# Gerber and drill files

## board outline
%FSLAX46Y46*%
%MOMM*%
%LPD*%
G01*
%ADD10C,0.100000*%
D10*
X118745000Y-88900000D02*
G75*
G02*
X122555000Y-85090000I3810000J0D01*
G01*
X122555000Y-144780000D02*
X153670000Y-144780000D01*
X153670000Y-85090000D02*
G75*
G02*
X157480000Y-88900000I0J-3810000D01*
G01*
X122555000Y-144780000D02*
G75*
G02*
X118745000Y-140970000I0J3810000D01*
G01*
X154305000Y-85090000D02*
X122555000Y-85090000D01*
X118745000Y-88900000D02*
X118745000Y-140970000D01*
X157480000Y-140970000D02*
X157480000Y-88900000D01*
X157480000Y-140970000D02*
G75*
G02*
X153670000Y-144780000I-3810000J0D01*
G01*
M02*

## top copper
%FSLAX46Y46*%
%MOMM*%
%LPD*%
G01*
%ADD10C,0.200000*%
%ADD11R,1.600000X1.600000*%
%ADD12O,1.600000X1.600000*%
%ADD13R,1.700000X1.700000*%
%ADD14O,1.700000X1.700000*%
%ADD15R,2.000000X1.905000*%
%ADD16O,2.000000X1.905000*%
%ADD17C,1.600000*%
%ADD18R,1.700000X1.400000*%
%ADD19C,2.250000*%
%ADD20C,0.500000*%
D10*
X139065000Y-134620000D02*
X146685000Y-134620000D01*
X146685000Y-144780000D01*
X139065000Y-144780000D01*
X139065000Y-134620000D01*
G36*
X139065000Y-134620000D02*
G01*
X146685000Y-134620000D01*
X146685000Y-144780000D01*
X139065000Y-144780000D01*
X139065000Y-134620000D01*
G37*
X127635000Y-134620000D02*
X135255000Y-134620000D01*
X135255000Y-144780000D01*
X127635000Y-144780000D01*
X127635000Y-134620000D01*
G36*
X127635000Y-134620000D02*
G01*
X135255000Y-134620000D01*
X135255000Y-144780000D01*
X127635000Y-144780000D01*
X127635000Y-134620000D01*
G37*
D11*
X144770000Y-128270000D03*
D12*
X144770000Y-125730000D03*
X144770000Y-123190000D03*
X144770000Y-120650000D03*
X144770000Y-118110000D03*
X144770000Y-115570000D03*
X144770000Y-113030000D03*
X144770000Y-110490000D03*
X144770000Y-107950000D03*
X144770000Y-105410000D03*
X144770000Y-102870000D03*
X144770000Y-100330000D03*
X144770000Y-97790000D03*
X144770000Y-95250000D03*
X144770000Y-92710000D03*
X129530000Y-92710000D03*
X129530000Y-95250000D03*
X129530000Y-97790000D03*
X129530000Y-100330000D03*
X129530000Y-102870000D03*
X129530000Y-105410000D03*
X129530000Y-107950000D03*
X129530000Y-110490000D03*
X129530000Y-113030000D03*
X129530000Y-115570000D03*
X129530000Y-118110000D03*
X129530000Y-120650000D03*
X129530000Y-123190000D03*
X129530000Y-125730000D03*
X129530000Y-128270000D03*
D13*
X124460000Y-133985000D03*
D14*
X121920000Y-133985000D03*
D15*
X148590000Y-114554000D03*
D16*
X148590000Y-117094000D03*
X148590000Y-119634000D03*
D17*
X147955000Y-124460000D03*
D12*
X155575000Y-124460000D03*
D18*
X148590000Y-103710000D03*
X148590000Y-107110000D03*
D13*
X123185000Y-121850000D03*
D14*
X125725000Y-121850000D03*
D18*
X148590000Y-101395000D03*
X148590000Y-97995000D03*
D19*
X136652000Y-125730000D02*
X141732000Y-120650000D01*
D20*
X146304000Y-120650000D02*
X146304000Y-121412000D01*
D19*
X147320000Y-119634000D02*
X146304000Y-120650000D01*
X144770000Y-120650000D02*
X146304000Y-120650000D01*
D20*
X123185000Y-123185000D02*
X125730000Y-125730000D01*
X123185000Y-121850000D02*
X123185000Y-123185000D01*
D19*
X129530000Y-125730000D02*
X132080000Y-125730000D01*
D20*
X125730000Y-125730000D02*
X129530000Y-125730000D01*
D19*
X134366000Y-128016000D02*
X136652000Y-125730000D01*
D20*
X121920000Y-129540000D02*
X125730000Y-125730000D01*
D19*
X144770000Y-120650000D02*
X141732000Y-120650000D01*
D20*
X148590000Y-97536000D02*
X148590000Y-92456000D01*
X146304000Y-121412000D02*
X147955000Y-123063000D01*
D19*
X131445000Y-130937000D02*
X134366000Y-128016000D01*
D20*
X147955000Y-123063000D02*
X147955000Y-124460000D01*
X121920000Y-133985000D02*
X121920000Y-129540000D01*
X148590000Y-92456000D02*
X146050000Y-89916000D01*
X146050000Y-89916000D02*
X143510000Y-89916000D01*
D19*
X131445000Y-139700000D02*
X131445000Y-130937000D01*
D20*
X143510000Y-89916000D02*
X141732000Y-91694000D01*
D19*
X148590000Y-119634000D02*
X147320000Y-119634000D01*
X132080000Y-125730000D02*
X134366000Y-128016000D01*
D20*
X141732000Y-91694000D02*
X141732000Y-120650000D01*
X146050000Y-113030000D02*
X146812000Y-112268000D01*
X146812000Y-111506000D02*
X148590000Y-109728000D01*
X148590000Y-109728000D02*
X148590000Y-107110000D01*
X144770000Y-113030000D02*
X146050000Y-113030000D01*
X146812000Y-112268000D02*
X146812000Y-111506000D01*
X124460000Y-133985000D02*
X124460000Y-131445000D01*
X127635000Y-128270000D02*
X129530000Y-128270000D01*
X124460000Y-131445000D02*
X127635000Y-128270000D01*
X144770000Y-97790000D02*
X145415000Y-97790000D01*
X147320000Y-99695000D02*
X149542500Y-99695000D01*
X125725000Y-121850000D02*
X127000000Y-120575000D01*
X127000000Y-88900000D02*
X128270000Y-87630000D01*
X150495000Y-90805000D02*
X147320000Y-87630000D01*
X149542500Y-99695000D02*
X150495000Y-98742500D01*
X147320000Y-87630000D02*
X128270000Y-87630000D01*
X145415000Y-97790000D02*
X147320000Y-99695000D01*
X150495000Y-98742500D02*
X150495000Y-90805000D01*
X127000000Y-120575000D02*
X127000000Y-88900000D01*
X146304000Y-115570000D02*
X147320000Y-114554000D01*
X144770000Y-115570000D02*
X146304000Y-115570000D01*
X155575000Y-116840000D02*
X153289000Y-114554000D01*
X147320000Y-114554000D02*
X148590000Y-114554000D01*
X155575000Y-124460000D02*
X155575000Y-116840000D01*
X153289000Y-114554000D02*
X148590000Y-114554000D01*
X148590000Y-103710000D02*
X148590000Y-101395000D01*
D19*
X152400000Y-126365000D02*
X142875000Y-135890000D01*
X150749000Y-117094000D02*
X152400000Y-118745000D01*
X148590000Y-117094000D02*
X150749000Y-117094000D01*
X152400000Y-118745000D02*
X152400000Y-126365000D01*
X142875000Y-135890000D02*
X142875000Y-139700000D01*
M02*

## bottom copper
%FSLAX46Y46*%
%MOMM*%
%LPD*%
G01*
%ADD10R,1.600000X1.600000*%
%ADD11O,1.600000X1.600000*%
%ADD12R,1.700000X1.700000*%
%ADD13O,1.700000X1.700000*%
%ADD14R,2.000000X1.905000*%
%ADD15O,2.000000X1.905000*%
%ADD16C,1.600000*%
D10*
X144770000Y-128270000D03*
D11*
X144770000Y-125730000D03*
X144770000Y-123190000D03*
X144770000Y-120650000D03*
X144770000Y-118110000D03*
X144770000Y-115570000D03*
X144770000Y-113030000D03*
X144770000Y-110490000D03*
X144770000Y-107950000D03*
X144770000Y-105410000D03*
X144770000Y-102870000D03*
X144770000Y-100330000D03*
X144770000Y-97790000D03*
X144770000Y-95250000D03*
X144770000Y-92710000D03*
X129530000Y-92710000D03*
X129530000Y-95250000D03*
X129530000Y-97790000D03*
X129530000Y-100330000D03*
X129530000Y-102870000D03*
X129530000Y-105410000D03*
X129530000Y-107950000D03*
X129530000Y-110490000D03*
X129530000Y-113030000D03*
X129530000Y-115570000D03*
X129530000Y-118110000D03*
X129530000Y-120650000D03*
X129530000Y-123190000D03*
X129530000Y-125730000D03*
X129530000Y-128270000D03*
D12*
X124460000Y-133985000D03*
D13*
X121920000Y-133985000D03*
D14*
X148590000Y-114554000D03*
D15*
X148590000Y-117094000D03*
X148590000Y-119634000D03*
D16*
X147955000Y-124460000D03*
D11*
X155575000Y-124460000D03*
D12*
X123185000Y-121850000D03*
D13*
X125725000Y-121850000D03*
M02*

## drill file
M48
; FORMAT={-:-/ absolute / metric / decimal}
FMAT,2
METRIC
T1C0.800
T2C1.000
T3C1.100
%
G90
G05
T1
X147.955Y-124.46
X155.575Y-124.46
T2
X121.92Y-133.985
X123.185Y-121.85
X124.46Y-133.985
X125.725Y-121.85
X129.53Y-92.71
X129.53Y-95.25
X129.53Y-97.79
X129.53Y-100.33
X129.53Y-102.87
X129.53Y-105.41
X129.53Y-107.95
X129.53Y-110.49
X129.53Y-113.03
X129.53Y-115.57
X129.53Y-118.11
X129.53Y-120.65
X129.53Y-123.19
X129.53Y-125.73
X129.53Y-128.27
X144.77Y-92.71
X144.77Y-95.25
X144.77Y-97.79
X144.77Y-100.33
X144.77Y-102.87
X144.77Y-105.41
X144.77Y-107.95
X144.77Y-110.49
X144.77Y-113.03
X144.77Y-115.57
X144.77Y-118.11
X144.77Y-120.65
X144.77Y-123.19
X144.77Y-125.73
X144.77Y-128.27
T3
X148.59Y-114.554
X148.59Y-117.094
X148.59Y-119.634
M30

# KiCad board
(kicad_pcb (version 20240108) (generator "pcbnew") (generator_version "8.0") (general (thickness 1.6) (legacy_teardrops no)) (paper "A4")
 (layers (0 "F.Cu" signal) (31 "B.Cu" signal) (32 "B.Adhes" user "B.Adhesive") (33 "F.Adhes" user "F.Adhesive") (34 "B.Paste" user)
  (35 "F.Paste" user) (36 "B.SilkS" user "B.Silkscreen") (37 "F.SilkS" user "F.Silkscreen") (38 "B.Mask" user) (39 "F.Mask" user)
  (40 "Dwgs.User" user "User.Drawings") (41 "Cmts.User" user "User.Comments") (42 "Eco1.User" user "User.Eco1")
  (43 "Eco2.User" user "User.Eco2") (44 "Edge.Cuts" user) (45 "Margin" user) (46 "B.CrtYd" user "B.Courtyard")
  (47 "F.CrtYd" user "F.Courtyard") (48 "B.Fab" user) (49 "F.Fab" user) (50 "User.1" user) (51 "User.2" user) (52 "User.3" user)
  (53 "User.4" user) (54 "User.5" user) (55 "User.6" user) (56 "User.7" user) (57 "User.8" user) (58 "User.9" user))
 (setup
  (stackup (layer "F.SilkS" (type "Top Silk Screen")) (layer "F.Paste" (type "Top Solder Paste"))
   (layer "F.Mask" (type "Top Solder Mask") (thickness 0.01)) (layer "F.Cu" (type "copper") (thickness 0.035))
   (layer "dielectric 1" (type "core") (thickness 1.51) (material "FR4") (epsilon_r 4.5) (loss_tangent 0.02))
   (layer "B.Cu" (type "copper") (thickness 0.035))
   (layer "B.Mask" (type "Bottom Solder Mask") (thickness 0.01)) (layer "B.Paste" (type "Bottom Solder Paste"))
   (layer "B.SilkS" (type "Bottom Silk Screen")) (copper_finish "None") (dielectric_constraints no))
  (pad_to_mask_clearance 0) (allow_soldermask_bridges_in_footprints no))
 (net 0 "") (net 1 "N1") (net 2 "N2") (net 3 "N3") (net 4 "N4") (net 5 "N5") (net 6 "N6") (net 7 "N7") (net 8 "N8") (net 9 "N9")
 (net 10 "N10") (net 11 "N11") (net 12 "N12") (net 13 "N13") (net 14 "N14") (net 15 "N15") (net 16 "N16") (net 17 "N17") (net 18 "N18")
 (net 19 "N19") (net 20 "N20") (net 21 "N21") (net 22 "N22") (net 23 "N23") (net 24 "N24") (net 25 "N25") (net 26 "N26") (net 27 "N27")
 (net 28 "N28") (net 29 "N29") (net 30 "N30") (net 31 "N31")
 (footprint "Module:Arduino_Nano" (layer "F.Cu") (at 144.77 128.27 180)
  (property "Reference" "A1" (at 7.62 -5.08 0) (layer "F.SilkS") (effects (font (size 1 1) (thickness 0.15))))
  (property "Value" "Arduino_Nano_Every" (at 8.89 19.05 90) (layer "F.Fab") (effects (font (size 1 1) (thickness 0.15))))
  (pad "1" thru_hole rect (at 0 0 180) (size 1.6 1.6) (drill 1) (layers "*.Cu" "*.Mask") (remove_unused_layers no) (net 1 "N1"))
  (pad "2" thru_hole oval (at 0 2.54 180) (size 1.6 1.6) (drill 1) (layers "*.Cu" "*.Mask") (remove_unused_layers no) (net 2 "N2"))
  (pad "3" thru_hole oval (at 0 5.08 180) (size 1.6 1.6) (drill 1) (layers "*.Cu" "*.Mask") (remove_unused_layers no) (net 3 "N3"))
  (pad "4" thru_hole oval (at 0 7.62 180) (size 1.6 1.6) (drill 1) (layers "*.Cu" "*.Mask") (remove_unused_layers no) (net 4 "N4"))
  (pad "5" thru_hole oval (at 0 10.16 180) (size 1.6 1.6) (drill 1) (layers "*.Cu" "*.Mask") (remove_unused_layers no) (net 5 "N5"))
  (pad "6" thru_hole oval (at 0 12.7 180) (size 1.6 1.6) (drill 1) (layers "*.Cu" "*.Mask") (remove_unused_layers no) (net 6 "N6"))
  (pad "7" thru_hole oval (at 0 15.24 180) (size 1.6 1.6) (drill 1) (layers "*.Cu" "*.Mask") (remove_unused_layers no) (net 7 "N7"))
  (pad "8" thru_hole oval (at 0 17.78 180) (size 1.6 1.6) (drill 1) (layers "*.Cu" "*.Mask") (remove_unused_layers no) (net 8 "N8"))
  (pad "9" thru_hole oval (at 0 20.32 180) (size 1.6 1.6) (drill 1) (layers "*.Cu" "*.Mask") (remove_unused_layers no) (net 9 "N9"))
  (pad "10" thru_hole oval (at 0 22.86 180) (size 1.6 1.6) (drill 1) (layers "*.Cu" "*.Mask") (remove_unused_layers no) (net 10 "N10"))
  (pad "11" thru_hole oval (at 0 25.4 180) (size 1.6 1.6) (drill 1) (layers "*.Cu" "*.Mask") (remove_unused_layers no) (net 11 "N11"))
  (pad "12" thru_hole oval (at 0 27.94 180) (size 1.6 1.6) (drill 1) (layers "*.Cu" "*.Mask") (remove_unused_layers no) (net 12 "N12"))
  (pad "13" thru_hole oval (at 0 30.48 180) (size 1.6 1.6) (drill 1) (layers "*.Cu" "*.Mask") (remove_unused_layers no) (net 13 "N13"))
  (pad "14" thru_hole oval (at 0 33.02 180) (size 1.6 1.6) (drill 1) (layers "*.Cu" "*.Mask") (remove_unused_layers no) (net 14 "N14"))
  (pad "15" thru_hole oval (at 0 35.56 180) (size 1.6 1.6) (drill 1) (layers "*.Cu" "*.Mask") (remove_unused_layers no) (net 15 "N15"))
  (pad "16" thru_hole oval (at 15.24 35.56 180) (size 1.6 1.6) (drill 1) (layers "*.Cu" "*.Mask") (remove_unused_layers no) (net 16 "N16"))
  (pad "17" thru_hole oval (at 15.24 33.02 180) (size 1.6 1.6) (drill 1) (layers "*.Cu" "*.Mask") (remove_unused_layers no) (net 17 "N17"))
  (pad "18" thru_hole oval (at 15.24 30.48 180) (size 1.6 1.6) (drill 1) (layers "*.Cu" "*.Mask") (remove_unused_layers no) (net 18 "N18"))
  (pad "19" thru_hole oval (at 15.24 27.94 180) (size 1.6 1.6) (drill 1) (layers "*.Cu" "*.Mask") (remove_unused_layers no) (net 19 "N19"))
  (pad "20" thru_hole oval (at 15.24 25.4 180) (size 1.6 1.6) (drill 1) (layers "*.Cu" "*.Mask") (remove_unused_layers no) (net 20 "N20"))
  (pad "21" thru_hole oval (at 15.24 22.86 180) (size 1.6 1.6) (drill 1) (layers "*.Cu" "*.Mask") (remove_unused_layers no) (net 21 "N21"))
  (pad "22" thru_hole oval (at 15.24 20.32 180) (size 1.6 1.6) (drill 1) (layers "*.Cu" "*.Mask") (remove_unused_layers no) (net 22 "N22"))
  (pad "23" thru_hole oval (at 15.24 17.78 180) (size 1.6 1.6) (drill 1) (layers "*.Cu" "*.Mask") (remove_unused_layers no) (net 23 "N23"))
  (pad "24" thru_hole oval (at 15.24 15.24 180) (size 1.6 1.6) (drill 1) (layers "*.Cu" "*.Mask") (remove_unused_layers no) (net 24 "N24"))
  (pad "25" thru_hole oval (at 15.24 12.7 180) (size 1.6 1.6) (drill 1) (layers "*.Cu" "*.Mask") (remove_unused_layers no) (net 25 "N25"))
  (pad "26" thru_hole oval (at 15.24 10.16 180) (size 1.6 1.6) (drill 1) (layers "*.Cu" "*.Mask") (remove_unused_layers no) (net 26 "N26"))
  (pad "27" thru_hole oval (at 15.24 7.62 180) (size 1.6 1.6) (drill 1) (layers "*.Cu" "*.Mask") (remove_unused_layers no) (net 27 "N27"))
  (pad "28" thru_hole oval (at 15.24 5.08 180) (size 1.6 1.6) (drill 1) (layers "*.Cu" "*.Mask") (remove_unused_layers no) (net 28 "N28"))
  (pad "29" thru_hole oval (at 15.24 2.54 180) (size 1.6 1.6) (drill 1) (layers "*.Cu" "*.Mask") (remove_unused_layers no) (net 4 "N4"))
  (pad "30" thru_hole oval (at 15.24 0 180) (size 1.6 1.6) (drill 1) (layers "*.Cu" "*.Mask") (remove_unused_layers no) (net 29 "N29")))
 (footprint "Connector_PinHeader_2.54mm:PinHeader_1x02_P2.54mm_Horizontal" (layer "F.Cu") (at 124.46 133.985 -90)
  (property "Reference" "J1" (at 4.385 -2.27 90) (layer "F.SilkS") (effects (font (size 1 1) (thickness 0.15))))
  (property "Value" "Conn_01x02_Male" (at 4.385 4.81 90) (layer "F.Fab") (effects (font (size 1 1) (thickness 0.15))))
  (pad "1" thru_hole rect (at 0 0 270) (size 1.7 1.7) (drill 1) (layers "*.Cu" "*.Mask") (remove_unused_layers no) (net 29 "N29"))
  (pad "2" thru_hole oval (at 0 2.54 270) (size 1.7 1.7) (drill 1) (layers "*.Cu" "*.Mask") (remove_unused_layers no) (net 4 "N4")))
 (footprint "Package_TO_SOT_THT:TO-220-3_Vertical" (layer "F.Cu") (at 148.59 114.554 -90)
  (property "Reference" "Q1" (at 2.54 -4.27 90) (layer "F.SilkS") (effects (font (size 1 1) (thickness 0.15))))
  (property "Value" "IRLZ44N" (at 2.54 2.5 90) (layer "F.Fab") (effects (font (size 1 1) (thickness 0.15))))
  (pad "1" thru_hole rect (at 0 0 270) (size 1.905 2) (drill 1.1) (layers "*.Cu" "*.Mask") (remove_unused_layers no) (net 6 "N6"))
  (pad "2" thru_hole oval (at 2.54 0 270) (size 1.905 2) (drill 1.1) (layers "*.Cu" "*.Mask") (remove_unused_layers no) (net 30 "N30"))
  (pad "3" thru_hole oval (at 5.08 0 270) (size 1.905 2) (drill 1.1) (layers "*.Cu" "*.Mask") (remove_unused_layers no) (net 4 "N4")))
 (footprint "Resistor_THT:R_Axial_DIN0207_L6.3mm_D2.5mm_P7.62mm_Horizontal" (layer "F.Cu") (at 147.955 124.46)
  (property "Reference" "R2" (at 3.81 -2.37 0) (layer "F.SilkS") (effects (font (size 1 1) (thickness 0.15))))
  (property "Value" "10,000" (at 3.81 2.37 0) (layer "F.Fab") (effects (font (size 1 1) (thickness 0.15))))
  (pad "1" thru_hole circle (at 0 0) (size 1.6 1.6) (drill 0.8) (layers "*.Cu" "*.Mask") (remove_unused_layers no) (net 4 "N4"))
  (pad "2" thru_hole oval (at 7.62 0) (size 1.6 1.6) (drill 0.8) (layers "*.Cu" "*.Mask") (remove_unused_layers no) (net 6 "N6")))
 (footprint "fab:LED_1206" (layer "F.Cu") (at 148.59 105.41 -90)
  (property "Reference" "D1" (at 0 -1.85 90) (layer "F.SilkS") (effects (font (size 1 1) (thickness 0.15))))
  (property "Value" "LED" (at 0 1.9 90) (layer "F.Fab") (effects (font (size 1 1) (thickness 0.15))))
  (pad "1" smd rect (at -1.7 0 270) (size 1.4 1.7) (layers "F.Cu" "F.Paste" "F.Mask") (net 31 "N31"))
  (pad "2" smd rect (at 1.7 0 270) (size 1.4 1.7) (layers "F.Cu" "F.Paste" "F.Mask") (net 7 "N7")))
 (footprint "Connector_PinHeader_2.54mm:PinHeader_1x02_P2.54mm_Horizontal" (layer "F.Cu") (at 123.185 121.85 90)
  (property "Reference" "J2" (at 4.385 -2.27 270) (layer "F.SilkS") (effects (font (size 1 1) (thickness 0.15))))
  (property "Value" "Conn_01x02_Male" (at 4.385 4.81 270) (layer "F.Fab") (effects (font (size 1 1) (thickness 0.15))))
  (pad "1" thru_hole rect (at 0 0 90) (size 1.7 1.7) (drill 1) (layers "*.Cu" "*.Mask") (remove_unused_layers no) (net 4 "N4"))
  (pad "2" thru_hole oval (at 0 2.54 90) (size 1.7 1.7) (drill 1) (layers "*.Cu" "*.Mask") (remove_unused_layers no) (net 13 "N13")))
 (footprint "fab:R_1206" (layer "F.Cu") (at 148.59 99.695 90)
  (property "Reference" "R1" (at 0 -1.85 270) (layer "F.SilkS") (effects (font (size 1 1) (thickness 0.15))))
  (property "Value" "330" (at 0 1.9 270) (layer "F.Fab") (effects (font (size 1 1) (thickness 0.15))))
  (pad "1" smd rect (at -1.7 0 90) (size 1.4 1.7) (layers "F.Cu" "F.Paste" "F.Mask") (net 31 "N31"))
  (pad "2" smd rect (at 1.7 0 90) (size 1.4 1.7) (layers "F.Cu" "F.Paste" "F.Mask") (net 4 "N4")))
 (gr_rect (start 139.065 134.62) (end 146.685 144.78) (stroke (width 0.2) (type solid)) (fill solid) (layer "F.Cu") (net 30))
 (gr_rect (start 127.635 134.62) (end 135.255 144.78) (stroke (width 0.2) (type solid)) (fill solid) (layer "F.Cu") (net 4))
 (gr_arc (start 118.745 88.9) (mid 119.860923 86.205923) (end 122.555 85.09) (stroke (width 0.1) (type default)) (layer "Edge.Cuts"))
 (gr_line (start 122.555 144.78) (end 153.67 144.78) (stroke (width 0.1) (type solid)) (layer "Edge.Cuts"))
 (gr_arc (start 153.67 85.09) (mid 156.364077 86.205923) (end 157.48 88.9) (stroke (width 0.1) (type solid)) (layer "Edge.Cuts"))
 (gr_arc (start 122.555 144.78) (mid 119.860923 143.664077) (end 118.745 140.97) (stroke (width 0.1) (type solid)) (layer "Edge.Cuts"))
 (gr_line (start 154.305 85.09) (end 122.555 85.09) (stroke (width 0.1) (type solid)) (layer "Edge.Cuts"))
 (gr_line (start 118.745 88.9) (end 118.745 140.97) (stroke (width 0.1) (type solid)) (layer "Edge.Cuts"))
 (gr_line (start 157.48 140.97) (end 157.48 88.9) (stroke (width 0.1) (type solid)) (layer "Edge.Cuts"))
 (gr_arc (start 157.48 140.97) (mid 156.364077 143.664077) (end 153.67 144.78) (stroke (width 0.1) (type solid)) (layer "Edge.Cuts"))
 (segment (start 136.652 125.73) (end 141.732 120.65) (width 2.25) (layer "F.Cu") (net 4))
 (segment (start 146.304 120.65) (end 146.304 121.412) (width 0.5) (layer "F.Cu") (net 4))
 (segment (start 147.32 119.634) (end 146.304 120.65) (width 2.25) (layer "F.Cu") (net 4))
 (segment (start 144.77 120.65) (end 146.304 120.65) (width 2.25) (layer "F.Cu") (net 4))
 (segment (start 123.185 123.185) (end 125.73 125.73) (width 0.5) (layer "F.Cu") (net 4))
 (segment (start 123.185 121.85) (end 123.185 123.185) (width 0.5) (layer "F.Cu") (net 4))
 (segment (start 129.53 125.73) (end 132.08 125.73) (width 2.25) (layer "F.Cu") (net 4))
 (segment (start 125.73 125.73) (end 129.53 125.73) (width 0.5) (layer "F.Cu") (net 4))
 (segment (start 134.366 128.016) (end 136.652 125.73) (width 2.25) (layer "F.Cu") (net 4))
 (segment (start 121.92 129.54) (end 125.73 125.73) (width 0.5) (layer "F.Cu") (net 4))
 (segment (start 144.77 120.65) (end 141.732 120.65) (width 2.25) (layer "F.Cu") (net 4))
 (segment (start 148.59 97.536) (end 148.59 92.456) (width 0.5) (layer "F.Cu") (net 4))
 (segment (start 146.304 121.412) (end 147.955 123.063) (width 0.5) (layer "F.Cu") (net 4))
 (segment (start 131.445 130.937) (end 134.366 128.016) (width 2.25) (layer "F.Cu") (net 4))
 (segment (start 147.955 123.063) (end 147.955 124.46) (width 0.5) (layer "F.Cu") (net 4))
 (segment (start 121.92 133.985) (end 121.92 129.54) (width 0.5) (layer "F.Cu") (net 4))
 (segment (start 148.59 92.456) (end 146.05 89.916) (width 0.5) (layer "F.Cu") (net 4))
 (segment (start 146.05 89.916) (end 143.51 89.916) (width 0.5) (layer "F.Cu") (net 4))
 (segment (start 131.445 139.7) (end 131.445 130.937) (width 2.25) (layer "F.Cu") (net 4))
 (segment (start 143.51 89.916) (end 141.732 91.694) (width 0.5) (layer "F.Cu") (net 4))
 (segment (start 148.59 119.634) (end 147.32 119.634) (width 2.25) (layer "F.Cu") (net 4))
 (segment (start 132.08 125.73) (end 134.366 128.016) (width 2.25) (layer "F.Cu") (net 4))
 (segment (start 141.732 91.694) (end 141.732 120.65) (width 0.5) (layer "F.Cu") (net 4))
 (segment (start 146.05 113.03) (end 146.812 112.268) (width 0.5) (layer "F.Cu") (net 7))
 (segment (start 146.812 111.506) (end 148.59 109.728) (width 0.5) (layer "F.Cu") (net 7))
 (segment (start 148.59 109.728) (end 148.59 107.11) (width 0.5) (layer "F.Cu") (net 7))
 (segment (start 144.77 113.03) (end 146.05 113.03) (width 0.5) (layer "F.Cu") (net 7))
 (segment (start 146.812 112.268) (end 146.812 111.506) (width 0.5) (layer "F.Cu") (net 7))
 (segment (start 124.46 133.985) (end 124.46 131.445) (width 0.5) (layer "F.Cu") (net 29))
 (segment (start 127.635 128.27) (end 129.53 128.27) (width 0.5) (layer "F.Cu") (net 29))
 (segment (start 124.46 131.445) (end 127.635 128.27) (width 0.5) (layer "F.Cu") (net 29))
 (segment (start 144.77 97.79) (end 145.415 97.79) (width 0.5) (layer "F.Cu") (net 13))
 (segment (start 147.32 99.695) (end 149.5425 99.695) (width 0.5) (layer "F.Cu") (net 13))
 (segment (start 125.725 121.85) (end 127 120.575) (width 0.5) (layer "F.Cu") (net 13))
 (segment (start 127 88.9) (end 128.27 87.63) (width 0.5) (layer "F.Cu") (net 13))
 (segment (start 150.495 90.805) (end 147.32 87.63) (width 0.5) (layer "F.Cu") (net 13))
 (segment (start 149.5425 99.695) (end 150.495 98.7425) (width 0.5) (layer "F.Cu") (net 13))
 (segment (start 147.32 87.63) (end 128.27 87.63) (width 0.5) (layer "F.Cu") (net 13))
 (segment (start 145.415 97.79) (end 147.32 99.695) (width 0.5) (layer "F.Cu") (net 13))
 (segment (start 150.495 98.7425) (end 150.495 90.805) (width 0.5) (layer "F.Cu") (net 13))
 (segment (start 127 120.575) (end 127 88.9) (width 0.5) (layer "F.Cu") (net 13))
 (segment (start 146.304 115.57) (end 147.32 114.554) (width 0.5) (layer "F.Cu") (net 6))
 (segment (start 144.77 115.57) (end 146.304 115.57) (width 0.5) (layer "F.Cu") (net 6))
 (segment (start 155.575 116.84) (end 153.289 114.554) (width 0.5) (layer "F.Cu") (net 6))
 (segment (start 147.32 114.554) (end 148.59 114.554) (width 0.5) (layer "F.Cu") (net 6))
 (segment (start 155.575 124.46) (end 155.575 116.84) (width 0.5) (layer "F.Cu") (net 6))
 (segment (start 153.289 114.554) (end 148.59 114.554) (width 0.5) (layer "F.Cu") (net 6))
 (segment (start 148.59 103.71) (end 148.59 101.395) (width 0.5) (layer "F.Cu") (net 31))
 (segment (start 152.4 126.365) (end 142.875 135.89) (width 2.25) (layer "F.Cu") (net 30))
 (segment (start 150.749 117.094) (end 152.4 118.745) (width 2.25) (layer "F.Cu") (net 30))
 (segment (start 148.59 117.094) (end 150.749 117.094) (width 2.25) (layer "F.Cu") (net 30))
 (segment (start 152.4 118.745) (end 152.4 126.365) (width 2.25) (layer "F.Cu") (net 30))
 (segment (start 142.875 135.89) (end 142.875 139.7) (width 2.25) (layer "F.Cu") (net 30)))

